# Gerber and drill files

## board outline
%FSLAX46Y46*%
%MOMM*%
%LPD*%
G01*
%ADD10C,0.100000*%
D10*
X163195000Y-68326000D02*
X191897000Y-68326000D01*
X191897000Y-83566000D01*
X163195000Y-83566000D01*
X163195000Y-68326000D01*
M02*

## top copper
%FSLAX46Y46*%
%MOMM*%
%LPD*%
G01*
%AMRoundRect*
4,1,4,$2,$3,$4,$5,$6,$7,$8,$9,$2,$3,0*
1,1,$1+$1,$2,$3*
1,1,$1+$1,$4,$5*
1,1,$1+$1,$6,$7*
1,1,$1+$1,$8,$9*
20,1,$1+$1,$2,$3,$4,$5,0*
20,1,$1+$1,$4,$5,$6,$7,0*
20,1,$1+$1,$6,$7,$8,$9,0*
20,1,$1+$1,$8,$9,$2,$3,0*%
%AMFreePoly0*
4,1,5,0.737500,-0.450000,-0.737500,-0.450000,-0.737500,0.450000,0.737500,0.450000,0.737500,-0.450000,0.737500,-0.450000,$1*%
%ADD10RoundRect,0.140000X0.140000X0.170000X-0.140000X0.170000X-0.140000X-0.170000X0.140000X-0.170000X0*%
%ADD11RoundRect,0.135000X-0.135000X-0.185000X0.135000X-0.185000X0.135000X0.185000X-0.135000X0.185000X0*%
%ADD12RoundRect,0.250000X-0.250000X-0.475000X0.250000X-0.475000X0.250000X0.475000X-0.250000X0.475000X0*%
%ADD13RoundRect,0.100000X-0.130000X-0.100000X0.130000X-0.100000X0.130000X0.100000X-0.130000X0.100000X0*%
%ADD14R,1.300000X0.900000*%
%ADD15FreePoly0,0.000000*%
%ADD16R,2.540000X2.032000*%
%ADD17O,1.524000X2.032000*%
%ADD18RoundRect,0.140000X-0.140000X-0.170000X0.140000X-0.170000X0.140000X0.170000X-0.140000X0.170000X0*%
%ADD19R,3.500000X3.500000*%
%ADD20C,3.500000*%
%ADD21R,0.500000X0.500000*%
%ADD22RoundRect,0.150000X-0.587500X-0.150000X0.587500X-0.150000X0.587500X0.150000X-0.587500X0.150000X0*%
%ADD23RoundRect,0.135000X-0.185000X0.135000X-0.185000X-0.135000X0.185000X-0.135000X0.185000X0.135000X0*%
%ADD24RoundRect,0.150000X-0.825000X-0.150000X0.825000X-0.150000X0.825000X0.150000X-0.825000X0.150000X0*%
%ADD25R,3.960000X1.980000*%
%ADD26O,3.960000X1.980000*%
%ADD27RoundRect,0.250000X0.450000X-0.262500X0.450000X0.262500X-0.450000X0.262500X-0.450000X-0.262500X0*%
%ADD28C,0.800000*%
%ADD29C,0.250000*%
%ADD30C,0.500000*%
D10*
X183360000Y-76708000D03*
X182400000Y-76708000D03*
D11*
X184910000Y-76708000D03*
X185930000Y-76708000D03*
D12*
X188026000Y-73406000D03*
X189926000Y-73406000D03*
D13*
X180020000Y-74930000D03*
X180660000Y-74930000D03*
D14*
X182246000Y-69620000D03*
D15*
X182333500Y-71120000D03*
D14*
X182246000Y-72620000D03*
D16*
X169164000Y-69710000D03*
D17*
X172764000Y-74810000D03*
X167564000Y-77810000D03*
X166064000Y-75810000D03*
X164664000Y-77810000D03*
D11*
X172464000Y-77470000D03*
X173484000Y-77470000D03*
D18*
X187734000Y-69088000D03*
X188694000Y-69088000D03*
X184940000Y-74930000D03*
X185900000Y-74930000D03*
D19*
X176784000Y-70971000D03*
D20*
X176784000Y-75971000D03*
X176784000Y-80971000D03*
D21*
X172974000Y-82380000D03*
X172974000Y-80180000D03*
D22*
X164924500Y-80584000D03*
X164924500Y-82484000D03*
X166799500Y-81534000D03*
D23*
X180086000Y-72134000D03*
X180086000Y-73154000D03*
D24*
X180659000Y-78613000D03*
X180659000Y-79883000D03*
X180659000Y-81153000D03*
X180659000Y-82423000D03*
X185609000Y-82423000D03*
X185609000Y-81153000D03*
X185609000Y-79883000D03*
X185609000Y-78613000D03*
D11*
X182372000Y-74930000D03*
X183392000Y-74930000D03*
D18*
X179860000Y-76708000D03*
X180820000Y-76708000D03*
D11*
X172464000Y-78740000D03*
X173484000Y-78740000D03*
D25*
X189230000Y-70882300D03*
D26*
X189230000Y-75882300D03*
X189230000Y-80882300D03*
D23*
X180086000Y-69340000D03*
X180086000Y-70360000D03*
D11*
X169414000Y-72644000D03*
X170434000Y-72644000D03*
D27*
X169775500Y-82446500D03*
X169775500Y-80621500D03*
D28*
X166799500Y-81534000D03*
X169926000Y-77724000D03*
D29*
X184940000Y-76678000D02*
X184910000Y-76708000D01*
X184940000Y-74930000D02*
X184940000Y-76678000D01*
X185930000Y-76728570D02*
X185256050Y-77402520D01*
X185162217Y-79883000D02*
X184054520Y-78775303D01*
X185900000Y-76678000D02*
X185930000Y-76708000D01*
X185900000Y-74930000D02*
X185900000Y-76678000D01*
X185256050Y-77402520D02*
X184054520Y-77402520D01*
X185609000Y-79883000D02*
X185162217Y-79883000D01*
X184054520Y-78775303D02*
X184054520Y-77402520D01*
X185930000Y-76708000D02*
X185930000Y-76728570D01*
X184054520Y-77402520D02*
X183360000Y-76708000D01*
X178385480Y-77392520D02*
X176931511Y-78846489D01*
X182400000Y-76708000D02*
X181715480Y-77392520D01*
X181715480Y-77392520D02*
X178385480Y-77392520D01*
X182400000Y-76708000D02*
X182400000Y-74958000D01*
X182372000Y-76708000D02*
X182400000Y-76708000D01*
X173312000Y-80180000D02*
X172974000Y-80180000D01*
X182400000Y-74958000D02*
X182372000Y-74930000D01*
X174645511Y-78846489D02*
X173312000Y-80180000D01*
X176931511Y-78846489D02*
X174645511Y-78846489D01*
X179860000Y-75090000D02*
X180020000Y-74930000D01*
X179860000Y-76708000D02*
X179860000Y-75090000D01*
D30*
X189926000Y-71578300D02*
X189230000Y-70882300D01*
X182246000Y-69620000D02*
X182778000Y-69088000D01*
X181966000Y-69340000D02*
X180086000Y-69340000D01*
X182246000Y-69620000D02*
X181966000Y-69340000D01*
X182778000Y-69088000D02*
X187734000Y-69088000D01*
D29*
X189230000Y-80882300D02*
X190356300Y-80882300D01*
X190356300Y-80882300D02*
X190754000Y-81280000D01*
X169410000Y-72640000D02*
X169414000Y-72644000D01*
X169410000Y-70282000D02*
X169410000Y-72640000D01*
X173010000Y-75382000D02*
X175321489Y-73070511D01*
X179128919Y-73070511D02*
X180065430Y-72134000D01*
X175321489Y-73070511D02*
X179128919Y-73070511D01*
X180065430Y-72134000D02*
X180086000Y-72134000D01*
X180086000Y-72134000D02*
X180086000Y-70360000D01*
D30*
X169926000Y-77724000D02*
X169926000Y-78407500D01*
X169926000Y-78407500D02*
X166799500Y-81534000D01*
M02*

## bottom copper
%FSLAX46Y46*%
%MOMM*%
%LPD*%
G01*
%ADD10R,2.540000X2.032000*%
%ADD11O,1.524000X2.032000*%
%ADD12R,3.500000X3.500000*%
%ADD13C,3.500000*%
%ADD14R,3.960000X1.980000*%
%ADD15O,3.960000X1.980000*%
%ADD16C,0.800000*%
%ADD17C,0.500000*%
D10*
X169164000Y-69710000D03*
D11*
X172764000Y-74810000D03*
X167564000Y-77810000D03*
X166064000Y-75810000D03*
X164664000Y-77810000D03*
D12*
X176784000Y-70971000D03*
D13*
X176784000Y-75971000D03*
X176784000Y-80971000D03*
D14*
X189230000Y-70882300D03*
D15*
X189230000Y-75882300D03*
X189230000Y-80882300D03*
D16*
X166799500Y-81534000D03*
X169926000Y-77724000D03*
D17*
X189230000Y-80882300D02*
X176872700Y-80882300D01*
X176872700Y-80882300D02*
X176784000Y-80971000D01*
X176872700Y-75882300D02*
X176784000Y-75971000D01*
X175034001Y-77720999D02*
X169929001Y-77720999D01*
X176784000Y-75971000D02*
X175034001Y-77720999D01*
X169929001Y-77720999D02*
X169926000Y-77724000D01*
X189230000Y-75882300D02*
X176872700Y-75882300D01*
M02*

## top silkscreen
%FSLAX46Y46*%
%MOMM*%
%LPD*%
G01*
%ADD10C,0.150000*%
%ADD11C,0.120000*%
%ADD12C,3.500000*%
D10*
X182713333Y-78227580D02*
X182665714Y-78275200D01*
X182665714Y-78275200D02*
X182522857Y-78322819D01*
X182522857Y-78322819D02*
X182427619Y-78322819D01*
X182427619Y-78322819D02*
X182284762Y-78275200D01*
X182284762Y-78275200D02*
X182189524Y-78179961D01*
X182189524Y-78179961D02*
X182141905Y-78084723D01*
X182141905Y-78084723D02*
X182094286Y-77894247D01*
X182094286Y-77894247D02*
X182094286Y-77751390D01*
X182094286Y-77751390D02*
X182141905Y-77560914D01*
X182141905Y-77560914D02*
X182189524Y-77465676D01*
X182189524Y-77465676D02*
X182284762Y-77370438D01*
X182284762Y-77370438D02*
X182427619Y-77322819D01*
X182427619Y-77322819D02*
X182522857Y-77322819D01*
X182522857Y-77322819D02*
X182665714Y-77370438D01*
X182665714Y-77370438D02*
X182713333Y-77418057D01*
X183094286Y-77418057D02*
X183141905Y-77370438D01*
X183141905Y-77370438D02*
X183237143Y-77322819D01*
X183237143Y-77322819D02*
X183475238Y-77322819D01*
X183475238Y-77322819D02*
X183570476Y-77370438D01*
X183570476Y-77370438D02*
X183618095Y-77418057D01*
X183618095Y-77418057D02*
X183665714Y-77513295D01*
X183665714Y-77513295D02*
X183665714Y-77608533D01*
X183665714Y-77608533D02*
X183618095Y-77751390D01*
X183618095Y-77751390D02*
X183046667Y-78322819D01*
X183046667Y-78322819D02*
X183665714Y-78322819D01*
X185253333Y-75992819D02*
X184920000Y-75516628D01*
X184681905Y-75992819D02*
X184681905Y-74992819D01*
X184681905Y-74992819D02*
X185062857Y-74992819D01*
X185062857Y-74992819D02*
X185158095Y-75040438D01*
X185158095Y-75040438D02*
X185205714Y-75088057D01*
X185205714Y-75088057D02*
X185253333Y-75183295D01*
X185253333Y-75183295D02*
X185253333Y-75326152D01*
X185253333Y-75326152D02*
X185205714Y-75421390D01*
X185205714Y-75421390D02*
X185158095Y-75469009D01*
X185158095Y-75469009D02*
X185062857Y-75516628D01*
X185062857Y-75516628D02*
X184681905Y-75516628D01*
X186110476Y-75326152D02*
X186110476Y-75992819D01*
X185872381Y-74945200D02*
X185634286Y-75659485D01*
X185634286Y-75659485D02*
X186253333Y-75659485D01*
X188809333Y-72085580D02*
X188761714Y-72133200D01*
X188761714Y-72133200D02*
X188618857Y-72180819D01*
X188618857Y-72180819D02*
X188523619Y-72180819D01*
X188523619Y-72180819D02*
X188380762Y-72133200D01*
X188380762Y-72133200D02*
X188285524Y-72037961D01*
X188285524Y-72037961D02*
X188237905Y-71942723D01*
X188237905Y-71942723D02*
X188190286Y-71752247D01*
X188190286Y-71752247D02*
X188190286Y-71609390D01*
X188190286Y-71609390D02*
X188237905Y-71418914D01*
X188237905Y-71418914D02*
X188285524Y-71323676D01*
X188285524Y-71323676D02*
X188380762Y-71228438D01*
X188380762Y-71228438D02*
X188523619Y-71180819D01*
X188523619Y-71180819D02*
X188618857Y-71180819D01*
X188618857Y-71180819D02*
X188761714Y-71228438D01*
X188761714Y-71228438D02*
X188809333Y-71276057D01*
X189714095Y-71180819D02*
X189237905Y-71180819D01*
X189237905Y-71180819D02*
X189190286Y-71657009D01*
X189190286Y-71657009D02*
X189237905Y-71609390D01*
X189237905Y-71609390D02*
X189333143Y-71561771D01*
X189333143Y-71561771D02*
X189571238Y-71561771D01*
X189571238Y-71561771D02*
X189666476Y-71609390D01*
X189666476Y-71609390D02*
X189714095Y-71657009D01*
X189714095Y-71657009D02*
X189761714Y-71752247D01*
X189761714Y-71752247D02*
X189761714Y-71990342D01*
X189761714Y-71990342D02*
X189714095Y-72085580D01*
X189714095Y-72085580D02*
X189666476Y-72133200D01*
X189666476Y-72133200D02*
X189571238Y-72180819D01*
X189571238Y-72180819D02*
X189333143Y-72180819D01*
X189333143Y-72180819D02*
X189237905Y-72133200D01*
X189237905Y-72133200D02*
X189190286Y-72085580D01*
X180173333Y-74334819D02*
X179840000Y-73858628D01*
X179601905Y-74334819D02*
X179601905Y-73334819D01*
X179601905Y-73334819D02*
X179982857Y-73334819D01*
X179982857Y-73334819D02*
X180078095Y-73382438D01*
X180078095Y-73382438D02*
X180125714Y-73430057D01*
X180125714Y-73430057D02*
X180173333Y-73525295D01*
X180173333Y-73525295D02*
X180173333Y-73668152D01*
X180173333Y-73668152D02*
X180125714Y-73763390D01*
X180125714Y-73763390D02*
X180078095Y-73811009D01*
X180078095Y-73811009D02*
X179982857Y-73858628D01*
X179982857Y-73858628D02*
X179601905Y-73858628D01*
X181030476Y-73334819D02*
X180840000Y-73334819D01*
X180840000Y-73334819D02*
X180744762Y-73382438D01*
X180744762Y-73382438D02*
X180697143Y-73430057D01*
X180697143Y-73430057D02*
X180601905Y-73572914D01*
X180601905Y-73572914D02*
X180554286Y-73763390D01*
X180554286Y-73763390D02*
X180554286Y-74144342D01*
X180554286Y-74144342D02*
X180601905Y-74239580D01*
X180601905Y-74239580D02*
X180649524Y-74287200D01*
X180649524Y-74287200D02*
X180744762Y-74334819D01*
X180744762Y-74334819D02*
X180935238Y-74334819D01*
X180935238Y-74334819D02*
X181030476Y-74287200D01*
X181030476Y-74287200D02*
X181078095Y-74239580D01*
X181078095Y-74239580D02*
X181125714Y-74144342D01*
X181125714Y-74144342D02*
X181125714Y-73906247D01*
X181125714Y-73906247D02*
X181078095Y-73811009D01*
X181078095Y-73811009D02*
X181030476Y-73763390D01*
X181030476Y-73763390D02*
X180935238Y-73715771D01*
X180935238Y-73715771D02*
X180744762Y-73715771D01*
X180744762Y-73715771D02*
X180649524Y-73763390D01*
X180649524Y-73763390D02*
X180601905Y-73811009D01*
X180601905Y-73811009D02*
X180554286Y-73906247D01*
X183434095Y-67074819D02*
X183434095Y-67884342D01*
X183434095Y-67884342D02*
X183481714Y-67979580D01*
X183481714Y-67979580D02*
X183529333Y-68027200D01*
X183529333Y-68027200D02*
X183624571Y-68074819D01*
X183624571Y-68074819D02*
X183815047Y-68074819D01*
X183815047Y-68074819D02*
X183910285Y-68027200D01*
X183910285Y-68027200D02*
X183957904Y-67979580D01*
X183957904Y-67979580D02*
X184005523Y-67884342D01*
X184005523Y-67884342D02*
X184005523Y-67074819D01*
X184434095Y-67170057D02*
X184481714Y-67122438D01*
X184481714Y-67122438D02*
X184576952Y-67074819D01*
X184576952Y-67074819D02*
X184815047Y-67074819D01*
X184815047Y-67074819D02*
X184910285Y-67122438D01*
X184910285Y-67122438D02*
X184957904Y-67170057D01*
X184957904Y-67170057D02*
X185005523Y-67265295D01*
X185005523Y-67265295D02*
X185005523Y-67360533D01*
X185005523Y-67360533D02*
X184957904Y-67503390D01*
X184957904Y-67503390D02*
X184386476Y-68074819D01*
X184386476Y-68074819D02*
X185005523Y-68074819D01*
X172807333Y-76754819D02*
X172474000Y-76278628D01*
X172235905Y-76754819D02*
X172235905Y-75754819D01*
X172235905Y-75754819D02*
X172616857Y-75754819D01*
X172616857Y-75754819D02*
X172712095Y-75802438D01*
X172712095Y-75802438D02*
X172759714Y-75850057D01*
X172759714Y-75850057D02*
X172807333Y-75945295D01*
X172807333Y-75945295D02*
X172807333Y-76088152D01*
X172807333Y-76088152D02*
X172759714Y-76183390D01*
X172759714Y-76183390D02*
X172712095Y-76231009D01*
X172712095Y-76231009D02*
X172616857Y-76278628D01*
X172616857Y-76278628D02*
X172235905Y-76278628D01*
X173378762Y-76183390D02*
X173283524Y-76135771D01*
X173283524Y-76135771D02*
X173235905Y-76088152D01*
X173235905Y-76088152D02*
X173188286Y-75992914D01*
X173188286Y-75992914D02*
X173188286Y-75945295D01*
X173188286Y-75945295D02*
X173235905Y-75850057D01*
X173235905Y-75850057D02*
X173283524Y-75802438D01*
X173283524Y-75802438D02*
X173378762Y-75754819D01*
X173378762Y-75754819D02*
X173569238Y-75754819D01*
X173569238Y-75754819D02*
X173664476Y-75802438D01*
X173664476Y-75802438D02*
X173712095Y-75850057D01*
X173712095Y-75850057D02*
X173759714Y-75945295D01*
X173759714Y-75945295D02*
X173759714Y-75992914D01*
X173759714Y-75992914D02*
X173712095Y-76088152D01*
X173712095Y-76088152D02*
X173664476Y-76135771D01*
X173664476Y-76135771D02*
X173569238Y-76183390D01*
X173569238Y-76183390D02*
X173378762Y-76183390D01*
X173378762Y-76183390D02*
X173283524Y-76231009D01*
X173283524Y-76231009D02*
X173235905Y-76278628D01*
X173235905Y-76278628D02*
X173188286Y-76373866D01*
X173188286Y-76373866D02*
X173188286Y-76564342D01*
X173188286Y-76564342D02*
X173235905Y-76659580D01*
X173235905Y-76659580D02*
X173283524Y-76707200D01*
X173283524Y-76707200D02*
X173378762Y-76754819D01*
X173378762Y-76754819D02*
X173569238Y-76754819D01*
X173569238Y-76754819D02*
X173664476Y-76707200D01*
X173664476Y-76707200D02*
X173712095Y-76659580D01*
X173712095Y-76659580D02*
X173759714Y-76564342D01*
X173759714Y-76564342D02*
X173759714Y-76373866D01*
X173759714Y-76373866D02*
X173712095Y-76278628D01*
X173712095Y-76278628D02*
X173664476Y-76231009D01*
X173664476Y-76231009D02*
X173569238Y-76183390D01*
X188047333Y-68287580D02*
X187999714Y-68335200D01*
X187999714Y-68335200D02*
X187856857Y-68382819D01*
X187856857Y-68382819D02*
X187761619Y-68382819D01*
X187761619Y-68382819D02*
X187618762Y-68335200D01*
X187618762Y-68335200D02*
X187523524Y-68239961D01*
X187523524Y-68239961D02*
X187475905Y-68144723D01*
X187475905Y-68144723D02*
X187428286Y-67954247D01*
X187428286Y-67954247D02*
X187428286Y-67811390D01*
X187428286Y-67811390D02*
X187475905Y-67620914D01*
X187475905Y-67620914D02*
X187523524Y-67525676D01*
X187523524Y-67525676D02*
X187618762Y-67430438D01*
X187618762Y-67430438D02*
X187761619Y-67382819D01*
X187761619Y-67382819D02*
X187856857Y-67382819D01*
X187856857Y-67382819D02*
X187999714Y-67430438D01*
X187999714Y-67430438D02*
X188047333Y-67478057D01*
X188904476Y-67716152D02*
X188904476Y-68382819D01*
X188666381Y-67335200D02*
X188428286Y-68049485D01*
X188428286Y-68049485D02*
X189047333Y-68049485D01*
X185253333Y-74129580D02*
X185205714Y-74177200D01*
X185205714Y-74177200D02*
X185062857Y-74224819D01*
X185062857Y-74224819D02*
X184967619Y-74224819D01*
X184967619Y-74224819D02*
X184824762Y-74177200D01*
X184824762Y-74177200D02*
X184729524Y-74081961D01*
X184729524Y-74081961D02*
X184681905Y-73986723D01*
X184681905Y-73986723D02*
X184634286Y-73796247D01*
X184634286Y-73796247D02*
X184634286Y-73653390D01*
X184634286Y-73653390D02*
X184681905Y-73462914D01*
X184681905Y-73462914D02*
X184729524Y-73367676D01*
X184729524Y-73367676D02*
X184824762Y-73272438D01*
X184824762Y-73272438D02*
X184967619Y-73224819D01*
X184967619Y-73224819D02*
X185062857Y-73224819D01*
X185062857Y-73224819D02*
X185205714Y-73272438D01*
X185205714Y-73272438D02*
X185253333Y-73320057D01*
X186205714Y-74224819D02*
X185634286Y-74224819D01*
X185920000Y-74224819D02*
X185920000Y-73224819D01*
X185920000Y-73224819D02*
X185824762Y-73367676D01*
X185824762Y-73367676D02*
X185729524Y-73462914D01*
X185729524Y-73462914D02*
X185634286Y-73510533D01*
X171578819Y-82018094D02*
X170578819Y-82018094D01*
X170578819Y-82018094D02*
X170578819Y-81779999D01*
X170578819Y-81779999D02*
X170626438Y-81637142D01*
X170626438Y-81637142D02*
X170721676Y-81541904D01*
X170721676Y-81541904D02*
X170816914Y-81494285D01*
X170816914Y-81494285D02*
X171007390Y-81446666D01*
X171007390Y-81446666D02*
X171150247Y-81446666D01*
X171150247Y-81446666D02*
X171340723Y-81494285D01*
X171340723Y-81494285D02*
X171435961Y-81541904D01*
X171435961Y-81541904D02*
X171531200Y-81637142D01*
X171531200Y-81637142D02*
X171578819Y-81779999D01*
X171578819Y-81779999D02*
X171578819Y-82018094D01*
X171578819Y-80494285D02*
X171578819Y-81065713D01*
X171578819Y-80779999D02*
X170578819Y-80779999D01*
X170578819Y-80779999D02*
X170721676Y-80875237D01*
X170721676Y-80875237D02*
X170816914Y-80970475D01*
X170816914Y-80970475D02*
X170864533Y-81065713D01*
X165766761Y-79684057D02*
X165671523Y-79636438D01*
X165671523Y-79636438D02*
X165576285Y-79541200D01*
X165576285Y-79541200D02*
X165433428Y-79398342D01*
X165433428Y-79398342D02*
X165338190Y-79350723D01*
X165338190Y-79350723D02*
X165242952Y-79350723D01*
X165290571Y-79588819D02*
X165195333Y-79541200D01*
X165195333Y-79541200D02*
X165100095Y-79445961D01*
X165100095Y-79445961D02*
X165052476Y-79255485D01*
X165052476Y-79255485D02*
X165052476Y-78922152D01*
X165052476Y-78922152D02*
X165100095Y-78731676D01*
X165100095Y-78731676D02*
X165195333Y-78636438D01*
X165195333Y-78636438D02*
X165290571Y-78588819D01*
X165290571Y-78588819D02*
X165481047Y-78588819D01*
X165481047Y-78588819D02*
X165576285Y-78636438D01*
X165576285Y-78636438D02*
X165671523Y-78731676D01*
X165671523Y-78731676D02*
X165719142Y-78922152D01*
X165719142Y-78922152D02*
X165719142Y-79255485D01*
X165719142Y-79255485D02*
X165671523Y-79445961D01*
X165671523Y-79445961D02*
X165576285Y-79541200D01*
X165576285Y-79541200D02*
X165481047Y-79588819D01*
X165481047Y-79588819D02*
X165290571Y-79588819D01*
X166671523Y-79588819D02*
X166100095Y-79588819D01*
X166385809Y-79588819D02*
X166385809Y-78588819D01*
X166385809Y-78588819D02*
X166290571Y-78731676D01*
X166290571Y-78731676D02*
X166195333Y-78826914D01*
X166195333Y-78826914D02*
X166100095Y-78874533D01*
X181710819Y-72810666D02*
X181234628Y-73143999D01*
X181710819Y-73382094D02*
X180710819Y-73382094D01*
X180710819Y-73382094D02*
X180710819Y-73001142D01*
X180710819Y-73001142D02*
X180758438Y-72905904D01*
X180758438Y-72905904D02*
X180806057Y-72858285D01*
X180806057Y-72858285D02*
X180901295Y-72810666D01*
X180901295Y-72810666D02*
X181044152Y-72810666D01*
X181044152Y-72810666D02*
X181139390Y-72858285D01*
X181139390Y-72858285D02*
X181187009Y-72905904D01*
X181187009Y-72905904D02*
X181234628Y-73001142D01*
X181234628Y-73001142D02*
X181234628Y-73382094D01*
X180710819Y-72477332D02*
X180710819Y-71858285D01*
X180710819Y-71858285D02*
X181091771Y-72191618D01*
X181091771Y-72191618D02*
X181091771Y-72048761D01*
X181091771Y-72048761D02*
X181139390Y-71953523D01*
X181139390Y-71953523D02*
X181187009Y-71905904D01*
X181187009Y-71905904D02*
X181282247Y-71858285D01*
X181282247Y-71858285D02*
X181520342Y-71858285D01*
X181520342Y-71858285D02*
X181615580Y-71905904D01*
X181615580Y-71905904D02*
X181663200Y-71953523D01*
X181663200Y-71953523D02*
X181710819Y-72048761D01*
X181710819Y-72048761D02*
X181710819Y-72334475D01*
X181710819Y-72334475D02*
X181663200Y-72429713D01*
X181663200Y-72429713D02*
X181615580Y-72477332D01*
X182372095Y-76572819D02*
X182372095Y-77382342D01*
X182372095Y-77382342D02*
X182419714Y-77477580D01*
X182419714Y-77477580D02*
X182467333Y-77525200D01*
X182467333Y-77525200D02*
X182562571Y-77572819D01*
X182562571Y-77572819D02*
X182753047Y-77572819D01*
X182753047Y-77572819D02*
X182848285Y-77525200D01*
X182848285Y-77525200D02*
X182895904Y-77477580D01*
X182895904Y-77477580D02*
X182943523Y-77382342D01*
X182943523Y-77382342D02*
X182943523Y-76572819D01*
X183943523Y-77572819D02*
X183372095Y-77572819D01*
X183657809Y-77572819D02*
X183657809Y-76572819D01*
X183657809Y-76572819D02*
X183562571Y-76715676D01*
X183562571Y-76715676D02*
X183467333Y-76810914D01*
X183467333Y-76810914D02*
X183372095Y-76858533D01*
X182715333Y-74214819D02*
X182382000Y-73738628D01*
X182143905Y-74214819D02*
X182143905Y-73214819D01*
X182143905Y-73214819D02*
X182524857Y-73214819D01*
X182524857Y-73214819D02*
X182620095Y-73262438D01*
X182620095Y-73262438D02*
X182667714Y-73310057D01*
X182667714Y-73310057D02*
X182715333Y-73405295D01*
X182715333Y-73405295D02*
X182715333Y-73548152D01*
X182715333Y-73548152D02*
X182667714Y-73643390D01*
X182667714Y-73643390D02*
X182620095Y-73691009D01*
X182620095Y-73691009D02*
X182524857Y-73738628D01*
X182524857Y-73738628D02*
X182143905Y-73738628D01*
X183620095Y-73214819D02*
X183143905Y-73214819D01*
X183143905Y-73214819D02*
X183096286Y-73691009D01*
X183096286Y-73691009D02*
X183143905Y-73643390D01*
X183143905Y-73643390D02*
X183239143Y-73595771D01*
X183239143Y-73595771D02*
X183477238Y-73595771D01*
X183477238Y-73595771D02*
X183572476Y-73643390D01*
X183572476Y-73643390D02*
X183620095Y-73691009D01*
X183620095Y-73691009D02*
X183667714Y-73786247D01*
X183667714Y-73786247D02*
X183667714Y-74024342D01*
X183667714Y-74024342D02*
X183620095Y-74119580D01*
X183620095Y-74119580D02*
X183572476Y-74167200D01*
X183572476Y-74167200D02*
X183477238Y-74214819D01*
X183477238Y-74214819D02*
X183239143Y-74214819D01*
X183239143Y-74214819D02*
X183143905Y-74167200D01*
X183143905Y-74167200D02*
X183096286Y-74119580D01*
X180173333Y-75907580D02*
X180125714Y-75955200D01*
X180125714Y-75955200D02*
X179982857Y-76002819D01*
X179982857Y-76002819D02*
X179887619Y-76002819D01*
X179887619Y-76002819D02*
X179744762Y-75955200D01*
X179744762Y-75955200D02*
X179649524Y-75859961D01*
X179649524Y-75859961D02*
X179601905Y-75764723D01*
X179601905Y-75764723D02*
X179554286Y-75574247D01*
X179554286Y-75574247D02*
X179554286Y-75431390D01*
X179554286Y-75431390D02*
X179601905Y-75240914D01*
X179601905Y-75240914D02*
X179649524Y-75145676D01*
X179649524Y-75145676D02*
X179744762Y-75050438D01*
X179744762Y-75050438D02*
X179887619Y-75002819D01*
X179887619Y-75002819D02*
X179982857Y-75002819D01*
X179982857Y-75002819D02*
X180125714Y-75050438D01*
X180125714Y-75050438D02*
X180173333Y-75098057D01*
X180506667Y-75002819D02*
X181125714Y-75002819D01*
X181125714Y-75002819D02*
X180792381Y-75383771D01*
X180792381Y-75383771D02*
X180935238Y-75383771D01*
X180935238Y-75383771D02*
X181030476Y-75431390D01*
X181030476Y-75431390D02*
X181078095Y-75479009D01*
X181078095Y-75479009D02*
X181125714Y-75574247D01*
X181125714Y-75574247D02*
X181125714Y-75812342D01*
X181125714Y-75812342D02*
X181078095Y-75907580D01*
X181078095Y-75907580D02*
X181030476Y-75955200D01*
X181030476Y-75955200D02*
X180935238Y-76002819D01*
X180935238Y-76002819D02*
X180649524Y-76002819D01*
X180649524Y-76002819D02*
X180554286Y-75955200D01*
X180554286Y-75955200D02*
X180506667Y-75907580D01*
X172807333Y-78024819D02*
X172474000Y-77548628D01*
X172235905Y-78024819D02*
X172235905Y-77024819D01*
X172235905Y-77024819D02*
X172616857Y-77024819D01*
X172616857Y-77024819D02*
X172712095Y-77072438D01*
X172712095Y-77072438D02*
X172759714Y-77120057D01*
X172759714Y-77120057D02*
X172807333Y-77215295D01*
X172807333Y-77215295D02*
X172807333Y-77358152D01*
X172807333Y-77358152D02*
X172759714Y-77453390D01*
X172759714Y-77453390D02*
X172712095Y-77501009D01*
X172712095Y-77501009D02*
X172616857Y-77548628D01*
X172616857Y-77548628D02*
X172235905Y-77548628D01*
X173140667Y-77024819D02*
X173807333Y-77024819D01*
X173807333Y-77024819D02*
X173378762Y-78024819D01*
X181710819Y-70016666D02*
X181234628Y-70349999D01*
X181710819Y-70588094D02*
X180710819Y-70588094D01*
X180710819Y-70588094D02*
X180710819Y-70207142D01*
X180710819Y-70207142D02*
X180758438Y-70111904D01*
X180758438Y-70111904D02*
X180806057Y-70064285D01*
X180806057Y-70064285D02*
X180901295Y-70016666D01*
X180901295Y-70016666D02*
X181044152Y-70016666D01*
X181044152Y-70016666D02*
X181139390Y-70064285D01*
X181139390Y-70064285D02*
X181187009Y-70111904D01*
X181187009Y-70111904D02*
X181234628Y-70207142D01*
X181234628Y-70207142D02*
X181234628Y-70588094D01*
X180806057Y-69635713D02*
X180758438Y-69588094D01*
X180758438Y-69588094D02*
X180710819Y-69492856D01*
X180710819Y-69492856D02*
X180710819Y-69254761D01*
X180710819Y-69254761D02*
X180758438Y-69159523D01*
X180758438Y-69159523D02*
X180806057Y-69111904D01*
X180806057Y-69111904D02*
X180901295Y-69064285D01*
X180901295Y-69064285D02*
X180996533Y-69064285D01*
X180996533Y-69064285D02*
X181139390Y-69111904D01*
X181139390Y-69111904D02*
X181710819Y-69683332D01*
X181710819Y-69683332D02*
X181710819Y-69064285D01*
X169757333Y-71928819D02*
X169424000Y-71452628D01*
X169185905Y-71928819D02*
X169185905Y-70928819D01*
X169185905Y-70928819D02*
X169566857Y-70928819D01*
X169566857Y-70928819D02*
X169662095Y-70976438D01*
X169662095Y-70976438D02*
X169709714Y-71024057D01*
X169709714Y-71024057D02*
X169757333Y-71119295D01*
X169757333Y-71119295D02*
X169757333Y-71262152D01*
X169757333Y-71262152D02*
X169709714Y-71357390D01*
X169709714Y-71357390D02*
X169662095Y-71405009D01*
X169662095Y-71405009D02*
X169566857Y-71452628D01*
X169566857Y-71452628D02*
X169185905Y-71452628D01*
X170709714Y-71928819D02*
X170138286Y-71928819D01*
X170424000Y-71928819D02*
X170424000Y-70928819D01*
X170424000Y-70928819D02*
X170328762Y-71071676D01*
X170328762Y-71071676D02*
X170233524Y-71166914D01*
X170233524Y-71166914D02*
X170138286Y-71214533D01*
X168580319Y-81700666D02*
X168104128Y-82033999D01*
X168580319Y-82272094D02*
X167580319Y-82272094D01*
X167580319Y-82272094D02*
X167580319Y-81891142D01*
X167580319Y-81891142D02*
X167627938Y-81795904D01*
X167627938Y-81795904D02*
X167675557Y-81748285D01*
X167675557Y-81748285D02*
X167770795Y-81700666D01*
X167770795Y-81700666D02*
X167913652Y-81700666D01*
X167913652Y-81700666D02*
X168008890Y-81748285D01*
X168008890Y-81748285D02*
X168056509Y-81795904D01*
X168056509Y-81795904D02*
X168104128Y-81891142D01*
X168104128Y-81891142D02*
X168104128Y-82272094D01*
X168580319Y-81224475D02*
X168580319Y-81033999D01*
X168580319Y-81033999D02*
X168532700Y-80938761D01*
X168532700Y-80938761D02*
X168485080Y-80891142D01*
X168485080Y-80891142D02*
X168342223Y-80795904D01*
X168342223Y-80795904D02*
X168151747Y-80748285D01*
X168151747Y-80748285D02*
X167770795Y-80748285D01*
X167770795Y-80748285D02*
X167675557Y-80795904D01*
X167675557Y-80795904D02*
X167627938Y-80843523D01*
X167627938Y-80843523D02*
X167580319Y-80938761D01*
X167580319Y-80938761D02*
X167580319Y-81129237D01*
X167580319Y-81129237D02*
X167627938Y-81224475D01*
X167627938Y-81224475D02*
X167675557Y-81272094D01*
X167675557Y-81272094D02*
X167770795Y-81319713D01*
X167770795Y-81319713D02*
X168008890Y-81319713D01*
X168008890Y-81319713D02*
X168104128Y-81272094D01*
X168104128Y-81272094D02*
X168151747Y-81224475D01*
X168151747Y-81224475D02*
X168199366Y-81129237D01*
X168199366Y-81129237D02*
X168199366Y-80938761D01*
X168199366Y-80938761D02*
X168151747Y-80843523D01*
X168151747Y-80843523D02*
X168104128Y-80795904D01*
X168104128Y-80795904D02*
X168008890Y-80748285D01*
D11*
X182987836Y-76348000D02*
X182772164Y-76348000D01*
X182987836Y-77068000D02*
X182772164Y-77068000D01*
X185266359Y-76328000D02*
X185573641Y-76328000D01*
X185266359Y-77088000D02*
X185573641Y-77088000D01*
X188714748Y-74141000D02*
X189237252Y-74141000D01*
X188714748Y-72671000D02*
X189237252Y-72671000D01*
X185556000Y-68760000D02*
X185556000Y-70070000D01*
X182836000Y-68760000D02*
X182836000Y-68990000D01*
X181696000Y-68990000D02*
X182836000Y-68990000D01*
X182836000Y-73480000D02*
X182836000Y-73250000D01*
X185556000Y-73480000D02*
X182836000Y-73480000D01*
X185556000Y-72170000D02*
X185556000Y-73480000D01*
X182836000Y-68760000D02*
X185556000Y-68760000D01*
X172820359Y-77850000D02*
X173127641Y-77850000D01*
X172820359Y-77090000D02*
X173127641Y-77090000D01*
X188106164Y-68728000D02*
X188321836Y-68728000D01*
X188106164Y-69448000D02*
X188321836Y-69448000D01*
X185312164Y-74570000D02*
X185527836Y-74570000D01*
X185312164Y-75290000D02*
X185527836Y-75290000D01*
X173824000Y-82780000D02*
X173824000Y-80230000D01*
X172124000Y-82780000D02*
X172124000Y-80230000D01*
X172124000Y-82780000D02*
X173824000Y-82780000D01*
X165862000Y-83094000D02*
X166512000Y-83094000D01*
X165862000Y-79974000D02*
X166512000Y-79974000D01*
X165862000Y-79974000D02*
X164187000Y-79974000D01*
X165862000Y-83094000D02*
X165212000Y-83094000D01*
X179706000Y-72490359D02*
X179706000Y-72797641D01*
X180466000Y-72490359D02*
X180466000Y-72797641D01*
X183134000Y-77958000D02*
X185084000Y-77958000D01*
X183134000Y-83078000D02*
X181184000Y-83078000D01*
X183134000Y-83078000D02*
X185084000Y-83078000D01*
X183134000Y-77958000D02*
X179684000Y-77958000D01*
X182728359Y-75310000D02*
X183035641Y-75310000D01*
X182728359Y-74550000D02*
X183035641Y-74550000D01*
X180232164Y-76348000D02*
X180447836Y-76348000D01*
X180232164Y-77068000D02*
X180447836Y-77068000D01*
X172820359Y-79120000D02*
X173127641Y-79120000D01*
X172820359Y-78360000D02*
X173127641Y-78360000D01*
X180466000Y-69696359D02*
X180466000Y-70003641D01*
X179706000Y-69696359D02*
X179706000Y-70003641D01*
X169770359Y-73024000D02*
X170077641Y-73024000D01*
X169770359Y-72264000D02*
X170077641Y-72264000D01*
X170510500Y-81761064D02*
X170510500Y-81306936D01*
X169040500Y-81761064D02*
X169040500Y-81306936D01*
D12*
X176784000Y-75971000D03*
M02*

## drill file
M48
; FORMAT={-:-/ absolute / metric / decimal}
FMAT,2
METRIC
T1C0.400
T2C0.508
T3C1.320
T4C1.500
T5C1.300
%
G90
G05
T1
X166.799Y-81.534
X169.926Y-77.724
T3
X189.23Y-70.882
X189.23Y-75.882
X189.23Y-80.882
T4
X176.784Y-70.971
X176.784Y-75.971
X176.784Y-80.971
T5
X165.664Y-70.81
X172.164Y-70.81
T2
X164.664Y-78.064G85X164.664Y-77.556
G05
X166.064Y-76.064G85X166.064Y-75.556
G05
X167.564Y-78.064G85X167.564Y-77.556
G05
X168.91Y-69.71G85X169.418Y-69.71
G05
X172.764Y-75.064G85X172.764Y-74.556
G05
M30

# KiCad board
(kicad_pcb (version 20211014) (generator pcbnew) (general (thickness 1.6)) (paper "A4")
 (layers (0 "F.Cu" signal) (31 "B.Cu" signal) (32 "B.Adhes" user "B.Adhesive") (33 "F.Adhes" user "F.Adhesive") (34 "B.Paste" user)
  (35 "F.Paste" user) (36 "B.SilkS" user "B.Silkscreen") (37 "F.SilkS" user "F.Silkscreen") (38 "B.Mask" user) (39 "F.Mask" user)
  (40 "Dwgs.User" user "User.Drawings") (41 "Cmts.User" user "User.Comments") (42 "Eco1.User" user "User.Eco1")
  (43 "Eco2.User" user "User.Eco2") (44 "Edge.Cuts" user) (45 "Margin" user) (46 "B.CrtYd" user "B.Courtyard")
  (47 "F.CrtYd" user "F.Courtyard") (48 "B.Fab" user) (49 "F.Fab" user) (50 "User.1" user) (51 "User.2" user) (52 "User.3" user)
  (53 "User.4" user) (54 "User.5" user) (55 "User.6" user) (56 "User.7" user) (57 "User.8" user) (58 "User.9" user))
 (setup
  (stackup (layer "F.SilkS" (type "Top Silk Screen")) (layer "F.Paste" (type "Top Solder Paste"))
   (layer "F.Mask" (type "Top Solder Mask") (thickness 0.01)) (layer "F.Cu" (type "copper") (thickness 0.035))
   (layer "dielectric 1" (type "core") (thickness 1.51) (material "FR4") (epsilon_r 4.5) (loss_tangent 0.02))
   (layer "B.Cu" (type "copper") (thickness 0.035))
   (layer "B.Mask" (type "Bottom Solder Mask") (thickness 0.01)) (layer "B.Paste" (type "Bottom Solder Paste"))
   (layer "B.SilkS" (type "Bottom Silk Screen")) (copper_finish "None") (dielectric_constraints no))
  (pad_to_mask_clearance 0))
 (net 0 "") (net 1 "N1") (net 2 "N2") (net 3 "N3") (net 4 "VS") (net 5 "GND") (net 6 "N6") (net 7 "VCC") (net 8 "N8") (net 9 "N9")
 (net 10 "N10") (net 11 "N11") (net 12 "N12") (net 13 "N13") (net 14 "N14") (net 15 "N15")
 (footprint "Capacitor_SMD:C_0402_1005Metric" (layer "F.Cu") (at 182.88 76.708 180)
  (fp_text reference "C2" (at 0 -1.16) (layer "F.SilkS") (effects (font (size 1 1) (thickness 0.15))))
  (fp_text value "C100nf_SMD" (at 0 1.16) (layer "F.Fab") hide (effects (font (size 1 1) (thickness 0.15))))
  (fp_line (start -0.107836 0.36) (end 0.107836 0.36) (layer "F.SilkS") (width 0.12))
  (fp_line (start -0.107836 -0.36) (end 0.107836 -0.36) (layer "F.SilkS") (width 0.12))
  (pad "1" smd roundrect locked (at -0.48 0 180) (size 0.56 0.62) (layers "F.Cu" "F.Paste" "F.Mask") (roundrect_rratio 0.25) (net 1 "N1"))
  (pad "2" smd roundrect locked (at 0.48 0 180) (size 0.56 0.62) (layers "F.Cu" "F.Paste" "F.Mask") (roundrect_rratio 0.25) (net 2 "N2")))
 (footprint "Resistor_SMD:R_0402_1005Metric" (layer "F.Cu") (at 185.42 76.708)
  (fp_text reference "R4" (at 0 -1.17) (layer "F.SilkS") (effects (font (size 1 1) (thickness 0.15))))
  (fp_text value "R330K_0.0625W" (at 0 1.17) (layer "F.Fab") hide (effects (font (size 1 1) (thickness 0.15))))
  (fp_line (start -0.153641 -0.38) (end 0.153641 -0.38) (layer "F.SilkS") (width 0.12))
  (fp_line (start -0.153641 0.38) (end 0.153641 0.38) (layer "F.SilkS") (width 0.12))
  (pad "1" smd roundrect locked (at -0.51 0) (size 0.54 0.64) (layers "F.Cu" "F.Paste" "F.Mask") (roundrect_rratio 0.25) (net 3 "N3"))
  (pad "2" smd roundrect locked (at 0.51 0) (size 0.54 0.64) (layers "F.Cu" "F.Paste" "F.Mask") (roundrect_rratio 0.25) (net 1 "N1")))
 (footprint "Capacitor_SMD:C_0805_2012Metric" (layer "F.Cu") (at 188.976 73.406)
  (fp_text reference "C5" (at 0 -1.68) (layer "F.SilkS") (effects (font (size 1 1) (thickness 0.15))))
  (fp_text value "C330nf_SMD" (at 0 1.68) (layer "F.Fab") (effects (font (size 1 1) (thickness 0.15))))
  (fp_line (start -0.261252 0.735) (end 0.261252 0.735) (layer "F.SilkS") (width 0.12))
  (fp_line (start -0.261252 -0.735) (end 0.261252 -0.735) (layer "F.SilkS") (width 0.12))
  (pad "1" smd roundrect locked (at -0.95 0) (size 1 1.45) (layers "F.Cu" "F.Paste" "F.Mask") (roundrect_rratio 0.25) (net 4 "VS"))
  (pad "2" smd roundrect locked (at 0.95 0) (size 1 1.45) (layers "F.Cu" "F.Paste" "F.Mask") (roundrect_rratio 0.25) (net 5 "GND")))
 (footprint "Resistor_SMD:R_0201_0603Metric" (layer "F.Cu") (at 180.34 74.93)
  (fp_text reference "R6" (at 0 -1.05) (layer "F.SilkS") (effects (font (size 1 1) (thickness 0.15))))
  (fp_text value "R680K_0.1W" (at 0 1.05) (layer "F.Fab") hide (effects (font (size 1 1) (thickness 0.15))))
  (pad "" smd roundrect locked (at 0.345 0) (size 0.318 0.36) (layers "F.Paste") (roundrect_rratio 0.25))
  (pad "" smd roundrect locked (at -0.345 0) (size 0.318 0.36) (layers "F.Paste") (roundrect_rratio 0.25))
  (pad "1" smd roundrect locked (at -0.32 0) (size 0.46 0.4) (layers "F.Cu" "F.Mask") (roundrect_rratio 0.25) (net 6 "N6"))
  (pad "2" smd roundrect locked (at 0.32 0) (size 0.46 0.4) (layers "F.Cu" "F.Mask") (roundrect_rratio 0.25) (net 5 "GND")))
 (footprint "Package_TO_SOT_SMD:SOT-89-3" (layer "F.Cu") (at 183.896 71.12)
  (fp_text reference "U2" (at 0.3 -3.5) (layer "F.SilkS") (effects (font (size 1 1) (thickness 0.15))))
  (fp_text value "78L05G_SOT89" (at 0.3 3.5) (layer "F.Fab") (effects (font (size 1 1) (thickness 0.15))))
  (fp_line (start 1.66 -2.36) (end 1.66 -1.05) (layer "F.SilkS") (width 0.12))
  (fp_line (start -1.06 -2.36) (end -1.06 -2.13) (layer "F.SilkS") (width 0.12))
  (fp_line (start -2.2 -2.13) (end -1.06 -2.13) (layer "F.SilkS") (width 0.12))
  (fp_line (start -1.06 2.36) (end -1.06 2.13) (layer "F.SilkS") (width 0.12))
  (fp_line (start 1.66 2.36) (end -1.06 2.36) (layer "F.SilkS") (width 0.12))
  (fp_line (start 1.66 1.05) (end 1.66 2.36) (layer "F.SilkS") (width 0.12))
  (fp_line (start -1.06 -2.36) (end 1.66 -2.36) (layer "F.SilkS") (width 0.12))
  (pad "1" smd rect locked (at -1.65 -1.5) (size 1.3 0.9) (layers "F.Cu" "F.Paste" "F.Mask") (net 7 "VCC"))
  (pad "2" smd custom locked (at -1.5625 0) (size 1.475 0.9) (layers "F.Cu" "F.Paste" "F.Mask") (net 5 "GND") (zone_connect 2)
   (options (clearance outline) (anchor rect)) (primitives))
  (pad "3" smd rect locked (at -1.65 1.5) (size 1.3 0.9) (layers "F.Cu" "F.Paste" "F.Mask") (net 4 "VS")))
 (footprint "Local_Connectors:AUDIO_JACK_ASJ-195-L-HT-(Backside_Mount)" (layer "F.Cu") (at 169.164 67.31 90)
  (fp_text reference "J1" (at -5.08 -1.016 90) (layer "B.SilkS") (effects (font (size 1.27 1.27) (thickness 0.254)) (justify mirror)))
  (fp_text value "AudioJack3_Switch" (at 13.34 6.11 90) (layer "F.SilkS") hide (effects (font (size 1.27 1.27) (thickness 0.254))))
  (pad "" np_thru_hole circle (at -3.5 -3.5 90) (size 1.3 1.3) (drill 1.3) (layers F&B.Cu *.Mask))
  (pad "" np_thru_hole circle (at -3.5 3 90) (size 1.3 1.3) (drill 1.3) (layers F&B.Cu *.Mask))
  (pad "1" thru_hole rect (at -2.4 0 90) (size 2.032 2.54) (drill oval 0.508 1.016) (layers *.Cu *.Mask) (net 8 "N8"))
  (pad "2" thru_hole oval (at -7.5 3.6 90) (size 2.032 1.524) (drill oval 1.016 0.508) (layers *.Cu *.Mask) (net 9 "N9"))
  (pad "3" thru_hole oval (at -10.5 -1.6 90) (size 2.032 1.524) (drill oval 1.016 0.508) (layers *.Cu *.Mask) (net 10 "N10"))
  (pad "5" thru_hole oval (at -8.5 -3.1 90) (size 2.032 1.524) (drill oval 1.016 0.508) (layers *.Cu *.Mask) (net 5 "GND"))
  (pad "6" thru_hole oval (at -10.5 -4.5 90) (size 2.032 1.524) (drill oval 1.016 0.508) (layers *.Cu *.Mask) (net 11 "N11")))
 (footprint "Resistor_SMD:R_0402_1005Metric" (layer "F.Cu") (at 172.974 77.47)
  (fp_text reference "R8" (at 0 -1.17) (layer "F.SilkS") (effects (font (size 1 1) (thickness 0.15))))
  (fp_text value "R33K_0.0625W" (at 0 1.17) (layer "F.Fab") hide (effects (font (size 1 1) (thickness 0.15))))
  (fp_line (start -0.153641 0.38) (end 0.153641 0.38) (layer "F.SilkS") (width 0.12))
  (fp_line (start -0.153641 -0.38) (end 0.153641 -0.38) (layer "F.SilkS") (width 0.12))
  (pad "1" smd roundrect locked (at -0.51 0) (size 0.54 0.64) (layers "F.Cu" "F.Paste" "F.Mask") (roundrect_rratio 0.25) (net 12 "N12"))
  (pad "2" smd roundrect locked (at 0.51 0) (size 0.54 0.64) (layers "F.Cu" "F.Paste" "F.Mask") (roundrect_rratio 0.25) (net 5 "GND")))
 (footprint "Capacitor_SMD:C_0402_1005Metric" (layer "F.Cu") (at 188.214 69.088)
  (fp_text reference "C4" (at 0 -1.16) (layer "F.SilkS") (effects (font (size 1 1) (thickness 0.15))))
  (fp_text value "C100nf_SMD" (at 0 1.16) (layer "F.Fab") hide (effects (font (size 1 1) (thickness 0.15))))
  (fp_line (start -0.107836 -0.36) (end 0.107836 -0.36) (layer "F.SilkS") (width 0.12))
  (fp_line (start -0.107836 0.36) (end 0.107836 0.36) (layer "F.SilkS") (width 0.12))
  (pad "1" smd roundrect locked (at -0.48 0) (size 0.56 0.62) (layers "F.Cu" "F.Paste" "F.Mask") (roundrect_rratio 0.25) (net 7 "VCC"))
  (pad "2" smd roundrect locked (at 0.48 0) (size 0.56 0.62) (layers "F.Cu" "F.Paste" "F.Mask") (roundrect_rratio 0.25) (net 5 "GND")))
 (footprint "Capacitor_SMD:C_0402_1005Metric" (layer "F.Cu") (at 185.42 74.93)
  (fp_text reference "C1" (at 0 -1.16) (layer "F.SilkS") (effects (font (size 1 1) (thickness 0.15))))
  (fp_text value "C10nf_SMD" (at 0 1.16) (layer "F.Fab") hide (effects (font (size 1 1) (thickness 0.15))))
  (fp_line (start -0.107836 -0.36) (end 0.107836 -0.36) (layer "F.SilkS") (width 0.12))
  (fp_line (start -0.107836 0.36) (end 0.107836 0.36) (layer "F.SilkS") (width 0.12))
  (pad "1" smd roundrect locked (at -0.48 0) (size 0.56 0.62) (layers "F.Cu" "F.Paste" "F.Mask") (roundrect_rratio 0.25) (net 3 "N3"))
  (pad "2" smd roundrect locked (at 0.48 0) (size 0.56 0.62) (layers "F.Cu" "F.Paste" "F.Mask") (roundrect_rratio 0.25) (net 1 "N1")))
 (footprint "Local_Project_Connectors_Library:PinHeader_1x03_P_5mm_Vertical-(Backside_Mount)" (layer "F.Cu") (at 176.784 70.971)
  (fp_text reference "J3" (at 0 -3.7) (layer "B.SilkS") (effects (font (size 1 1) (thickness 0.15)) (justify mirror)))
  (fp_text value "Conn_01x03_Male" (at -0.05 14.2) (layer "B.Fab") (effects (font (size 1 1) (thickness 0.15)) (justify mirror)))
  (pad "1" thru_hole rect (at 0 0) (size 3.5 3.5) (drill 1.5) (layers *.Cu *.Mask) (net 5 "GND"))
  (pad "2" thru_hole circle (at 0 5) (size 3.5 3.5) (drill 1.5) (layers *.Cu *.Mask "F.SilkS") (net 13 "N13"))
  (pad "3" thru_hole circle (at 0 10) (size 3.5 3.5) (drill 1.5) (layers *.Cu *.Mask) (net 4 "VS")))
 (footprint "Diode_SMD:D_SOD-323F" (layer "F.Cu") (at 172.974 81.28 90)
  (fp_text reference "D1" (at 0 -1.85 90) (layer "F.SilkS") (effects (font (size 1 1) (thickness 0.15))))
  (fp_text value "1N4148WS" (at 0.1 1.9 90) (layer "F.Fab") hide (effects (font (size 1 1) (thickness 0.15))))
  (fp_line (start -1.5 0.85) (end 1.05 0.85) (layer "F.SilkS") (width 0.12))
  (fp_line (start -1.5 -0.85) (end 1.05 -0.85) (layer "F.SilkS") (width 0.12))
  (fp_line (start -1.5 -0.85) (end -1.5 0.85) (layer "F.SilkS") (width 0.12))
  (pad "1" smd rect locked (at -1.1 0 90) (size 0.5 0.5) (layers "F.Cu" "F.Paste" "F.Mask") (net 6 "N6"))
  (pad "2" smd rect locked (at 1.1 0 90) (size 0.5 0.5) (layers "F.Cu" "F.Paste" "F.Mask") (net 2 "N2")))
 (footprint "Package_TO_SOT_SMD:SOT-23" (layer "F.Cu") (at 165.862 81.534)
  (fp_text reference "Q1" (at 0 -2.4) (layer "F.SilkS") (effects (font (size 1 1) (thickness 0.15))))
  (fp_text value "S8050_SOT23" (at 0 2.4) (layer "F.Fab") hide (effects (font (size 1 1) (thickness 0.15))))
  (fp_line (start 0 1.56) (end 0.65 1.56) (layer "F.SilkS") (width 0.12))
  (fp_line (start 0 -1.56) (end 0.65 -1.56) (layer "F.SilkS") (width 0.12))
  (fp_line (start 0 -1.56) (end -1.675 -1.56) (layer "F.SilkS") (width 0.12))
  (fp_line (start 0 1.56) (end -0.65 1.56) (layer "F.SilkS") (width 0.12))
  (pad "1" smd roundrect locked (at -0.9375 -0.95) (size 1.475 0.6) (layers "F.Cu" "F.Paste" "F.Mask") (roundrect_rratio 0.25)
   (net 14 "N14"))
  (pad "2" smd roundrect locked (at -0.9375 0.95) (size 1.475 0.6) (layers "F.Cu" "F.Paste" "F.Mask") (roundrect_rratio 0.25) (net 5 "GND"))
  (pad "3" smd roundrect locked (at 0.9375 0) (size 1.475 0.6) (layers "F.Cu" "F.Paste" "F.Mask") (roundrect_rratio 0.25) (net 13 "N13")))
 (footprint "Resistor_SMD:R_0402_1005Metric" (layer "F.Cu") (at 180.086 72.644 -90)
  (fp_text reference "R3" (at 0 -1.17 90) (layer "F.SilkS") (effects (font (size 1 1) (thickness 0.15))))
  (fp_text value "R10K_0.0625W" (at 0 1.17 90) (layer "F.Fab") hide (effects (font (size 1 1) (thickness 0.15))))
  (fp_line (start -0.153641 0.38) (end 0.153641 0.38) (layer "F.SilkS") (width 0.12))
  (fp_line (start -0.153641 -0.38) (end 0.153641 -0.38) (layer "F.SilkS") (width 0.12))
  (pad "1" smd roundrect locked (at -0.51 0 270) (size 0.54 0.64) (layers "F.Cu" "F.Paste" "F.Mask") (roundrect_rratio 0.25) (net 9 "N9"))
  (pad "2" smd roundrect locked (at 0.51 0 270) (size 0.54 0.64) (layers "F.Cu" "F.Paste" "F.Mask") (roundrect_rratio 0.25) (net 5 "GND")))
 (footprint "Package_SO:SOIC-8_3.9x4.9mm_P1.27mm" (layer "F.Cu") (at 183.134 80.518)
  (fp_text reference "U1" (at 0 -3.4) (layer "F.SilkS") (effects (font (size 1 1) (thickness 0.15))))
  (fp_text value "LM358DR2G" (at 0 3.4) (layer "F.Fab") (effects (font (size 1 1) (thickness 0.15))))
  (fp_line (start 0 -2.56) (end 1.95 -2.56) (layer "F.SilkS") (width 0.12))
  (fp_line (start 0 2.56) (end -1.95 2.56) (layer "F.SilkS") (width 0.12))
  (fp_line (start 0 2.56) (end 1.95 2.56) (layer "F.SilkS") (width 0.12))
  (fp_line (start 0 -2.56) (end -3.45 -2.56) (layer "F.SilkS") (width 0.12))
  (pad "1" smd roundrect locked (at -2.475 -1.905) (size 1.95 0.6) (layers "F.Cu" "F.Paste" "F.Mask") (roundrect_rratio 0.25) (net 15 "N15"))
  (pad "2" smd roundrect locked (at -2.475 -0.635) (size 1.95 0.6) (layers "F.Cu" "F.Paste" "F.Mask") (roundrect_rratio 0.25) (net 12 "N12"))
  (pad "3" smd roundrect locked (at -2.475 0.635) (size 1.95 0.6) (layers "F.Cu" "F.Paste" "F.Mask") (roundrect_rratio 0.25) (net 6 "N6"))
  (pad "4" smd roundrect locked (at -2.475 1.905) (size 1.95 0.6) (layers "F.Cu" "F.Paste" "F.Mask") (roundrect_rratio 0.25) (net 5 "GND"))
  (pad "5" smd roundrect locked (at 2.475 1.905) (size 1.95 0.6) (layers "F.Cu" "F.Paste" "F.Mask") (roundrect_rratio 0.25) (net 3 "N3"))
  (pad "6" smd roundrect locked (at 2.475 0.635) (size 1.95 0.6) (layers "F.Cu" "F.Paste" "F.Mask") (roundrect_rratio 0.25) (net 9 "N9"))
  (pad "7" smd roundrect locked (at 2.475 -0.635) (size 1.95 0.6) (layers "F.Cu" "F.Paste" "F.Mask") (roundrect_rratio 0.25) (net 1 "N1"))
  (pad "8" smd roundrect locked (at 2.475 -1.905) (size 1.95 0.6) (layers "F.Cu" "F.Paste" "F.Mask") (roundrect_rratio 0.25) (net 7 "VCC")))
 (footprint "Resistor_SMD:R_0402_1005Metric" (layer "F.Cu") (at 182.882 74.93)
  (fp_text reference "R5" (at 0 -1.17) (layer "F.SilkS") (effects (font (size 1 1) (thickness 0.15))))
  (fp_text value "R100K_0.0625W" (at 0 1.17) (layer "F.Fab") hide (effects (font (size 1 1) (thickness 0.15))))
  (fp_line (start -0.153641 0.38) (end 0.153641 0.38) (layer "F.SilkS") (width 0.12))
  (fp_line (start -0.153641 -0.38) (end 0.153641 -0.38) (layer "F.SilkS") (width 0.12))
  (pad "1" smd roundrect locked (at -0.51 0) (size 0.54 0.64) (layers "F.Cu" "F.Paste" "F.Mask") (roundrect_rratio 0.25) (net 2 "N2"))
  (pad "2" smd roundrect locked (at 0.51 0) (size 0.54 0.64) (layers "F.Cu" "F.Paste" "F.Mask") (roundrect_rratio 0.25) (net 5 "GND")))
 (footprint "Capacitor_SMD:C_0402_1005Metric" (layer "F.Cu") (at 180.34 76.708)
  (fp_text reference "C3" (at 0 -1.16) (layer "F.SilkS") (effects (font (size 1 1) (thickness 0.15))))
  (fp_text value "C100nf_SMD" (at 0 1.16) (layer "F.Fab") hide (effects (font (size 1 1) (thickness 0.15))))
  (fp_line (start -0.107836 -0.36) (end 0.107836 -0.36) (layer "F.SilkS") (width 0.12))
  (fp_line (start -0.107836 0.36) (end 0.107836 0.36) (layer "F.SilkS") (width 0.12))
  (pad "1" smd roundrect locked (at -0.48 0) (size 0.56 0.62) (layers "F.Cu" "F.Paste" "F.Mask") (roundrect_rratio 0.25) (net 6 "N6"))
  (pad "2" smd roundrect locked (at 0.48 0) (size 0.56 0.62) (layers "F.Cu" "F.Paste" "F.Mask") (roundrect_rratio 0.25) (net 5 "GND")))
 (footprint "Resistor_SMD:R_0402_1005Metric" (layer "F.Cu") (at 172.974 78.74)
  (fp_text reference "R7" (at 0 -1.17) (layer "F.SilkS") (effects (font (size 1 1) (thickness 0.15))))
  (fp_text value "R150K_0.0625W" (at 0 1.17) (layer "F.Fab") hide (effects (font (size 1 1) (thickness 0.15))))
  (fp_line (start -0.153641 0.38) (end 0.153641 0.38) (layer "F.SilkS") (width 0.12))
  (fp_line (start -0.153641 -0.38) (end 0.153641 -0.38) (layer "F.SilkS") (width 0.12))
  (pad "1" smd roundrect locked (at -0.51 0) (size 0.54 0.64) (layers "F.Cu" "F.Paste" "F.Mask") (roundrect_rratio 0.25) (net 7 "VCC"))
  (pad "2" smd roundrect locked (at 0.51 0) (size 0.54 0.64) (layers "F.Cu" "F.Paste" "F.Mask") (roundrect_rratio 0.25) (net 12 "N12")))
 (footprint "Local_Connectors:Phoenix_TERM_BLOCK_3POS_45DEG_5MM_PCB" (layer "F.Cu") (at 189.23 70.8823 -90)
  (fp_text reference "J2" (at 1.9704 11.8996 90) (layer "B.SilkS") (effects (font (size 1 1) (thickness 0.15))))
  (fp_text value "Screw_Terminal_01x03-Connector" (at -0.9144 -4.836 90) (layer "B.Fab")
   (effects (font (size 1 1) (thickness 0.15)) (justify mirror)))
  (pad "1" thru_hole rect locked (at 0 0 270) (size 1.98 3.96) (drill 1.32) (layers *.Cu *.Mask "F.Paste") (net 5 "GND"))
  (pad "2" thru_hole oval locked (at 5 0 270) (size 1.98 3.96) (drill 1.32) (layers *.Cu *.Mask "F.Paste") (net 13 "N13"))
  (pad "3" thru_hole oval locked (at 10 0 270) (size 1.98 3.96) (drill 1.32) (layers *.Cu *.Mask "F.Paste") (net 4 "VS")))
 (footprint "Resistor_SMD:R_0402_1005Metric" (layer "F.Cu") (at 180.086 69.85 -90)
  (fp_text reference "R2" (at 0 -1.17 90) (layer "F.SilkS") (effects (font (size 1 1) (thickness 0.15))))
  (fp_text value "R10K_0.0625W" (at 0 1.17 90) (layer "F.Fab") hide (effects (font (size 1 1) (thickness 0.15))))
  (fp_line (start -0.153641 -0.38) (end 0.153641 -0.38) (layer "F.SilkS") (width 0.12))
  (fp_line (start -0.153641 0.38) (end 0.153641 0.38) (layer "F.SilkS") (width 0.12))
  (pad "1" smd roundrect locked (at -0.51 0 270) (size 0.54 0.64) (layers "F.Cu" "F.Paste" "F.Mask") (roundrect_rratio 0.25) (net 7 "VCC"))
  (pad "2" smd roundrect locked (at 0.51 0 270) (size 0.54 0.64) (layers "F.Cu" "F.Paste" "F.Mask") (roundrect_rratio 0.25) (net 9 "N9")))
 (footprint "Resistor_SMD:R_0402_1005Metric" (layer "F.Cu") (at 169.924 72.644)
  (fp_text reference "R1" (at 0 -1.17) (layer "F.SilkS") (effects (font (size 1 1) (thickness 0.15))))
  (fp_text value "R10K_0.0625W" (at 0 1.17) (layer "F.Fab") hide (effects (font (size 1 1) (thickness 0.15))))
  (fp_line (start -0.153641 0.38) (end 0.153641 0.38) (layer "F.SilkS") (width 0.12))
  (fp_line (start -0.153641 -0.38) (end 0.153641 -0.38) (layer "F.SilkS") (width 0.12))
  (pad "1" smd roundrect locked (at -0.51 0) (size 0.54 0.64) (layers "F.Cu" "F.Paste" "F.Mask") (roundrect_rratio 0.25) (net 8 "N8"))
  (pad "2" smd roundrect locked (at 0.51 0) (size 0.54 0.64) (layers "F.Cu" "F.Paste" "F.Mask") (roundrect_rratio 0.25) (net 3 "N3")))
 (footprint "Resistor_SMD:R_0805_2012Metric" (layer "F.Cu") (at 169.7755 81.534 90)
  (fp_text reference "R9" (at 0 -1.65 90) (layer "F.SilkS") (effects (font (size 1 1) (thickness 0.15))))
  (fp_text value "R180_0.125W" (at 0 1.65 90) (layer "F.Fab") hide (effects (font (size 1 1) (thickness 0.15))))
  (fp_line (start -0.227064 0.735) (end 0.227064 0.735) (layer "F.SilkS") (width 0.12))
  (fp_line (start -0.227064 -0.735) (end 0.227064 -0.735) (layer "F.SilkS") (width 0.12))
  (pad "1" smd roundrect locked (at -0.9125 0 90) (size 1.025 1.4) (layers "F.Cu" "F.Paste" "F.Mask") (roundrect_rratio 0.243902)
   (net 15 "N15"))
  (pad "2" smd roundrect locked (at 0.9125 0 90) (size 1.025 1.4) (layers "F.Cu" "F.Paste" "F.Mask") (roundrect_rratio 0.243902)
   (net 14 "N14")))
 (gr_rect (start 191.897 83.566) (end 163.195 68.326) (layer "Edge.Cuts") (width 0.1) (fill none))
 (segment (start 184.94 76.678) (end 184.91 76.708) (width 0.25) (layer "F.Cu") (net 3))
 (segment (start 184.94 74.93) (end 184.94 76.678) (width 0.25) (layer "F.Cu") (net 3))
 (segment (start 185.93 76.72857) (end 185.25605 77.40252) (width 0.25) (layer "F.Cu") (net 1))
 (segment (start 185.162217 79.883) (end 184.05452 78.775303) (width 0.25) (layer "F.Cu") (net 1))
 (segment (start 185.9 76.678) (end 185.93 76.708) (width 0.25) (layer "F.Cu") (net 1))
 (segment (start 185.9 74.93) (end 185.9 76.678) (width 0.25) (layer "F.Cu") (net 1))
 (segment (start 185.25605 77.40252) (end 184.05452 77.40252) (width 0.25) (layer "F.Cu") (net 1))
 (segment (start 185.609 79.883) (end 185.162217 79.883) (width 0.25) (layer "F.Cu") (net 1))
 (segment (start 184.05452 78.775303) (end 184.05452 77.40252) (width 0.25) (layer "F.Cu") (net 1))
 (segment (start 185.93 76.708) (end 185.93 76.72857) (width 0.25) (layer "F.Cu") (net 1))
 (segment (start 184.05452 77.40252) (end 183.36 76.708) (width 0.25) (layer "F.Cu") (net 1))
 (segment (start 178.38548 77.39252) (end 176.931511 78.846489) (width 0.25) (layer "F.Cu") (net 2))
 (segment (start 182.4 76.708) (end 181.71548 77.39252) (width 0.25) (layer "F.Cu") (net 2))
 (segment (start 181.71548 77.39252) (end 178.38548 77.39252) (width 0.25) (layer "F.Cu") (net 2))
 (segment (start 182.4 76.708) (end 182.4 74.958) (width 0.25) (layer "F.Cu") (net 2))
 (segment (start 182.372 76.708) (end 182.4 76.708) (width 0.25) (layer "F.Cu") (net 2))
 (segment (start 173.312 80.18) (end 172.974 80.18) (width 0.25) (layer "F.Cu") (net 2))
 (segment (start 182.4 74.958) (end 182.372 74.93) (width 0.25) (layer "F.Cu") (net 2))
 (segment (start 174.645511 78.846489) (end 173.312 80.18) (width 0.25) (layer "F.Cu") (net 2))
 (segment (start 176.931511 78.846489) (end 174.645511 78.846489) (width 0.25) (layer "F.Cu") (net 2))
 (segment (start 179.86 75.09) (end 180.02 74.93) (width 0.25) (layer "F.Cu") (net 6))
 (segment (start 179.86 76.708) (end 179.86 75.09) (width 0.25) (layer "F.Cu") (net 6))
 (segment (start 189.926 71.5783) (end 189.23 70.8823) (width 0.5) (layer "F.Cu") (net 5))
 (segment (start 182.246 69.62) (end 182.778 69.088) (width 0.5) (layer "F.Cu") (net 7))
 (segment (start 181.966 69.34) (end 180.086 69.34) (width 0.5) (layer "F.Cu") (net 7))
 (segment (start 182.246 69.62) (end 181.966 69.34) (width 0.5) (layer "F.Cu") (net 7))
 (segment (start 182.778 69.088) (end 187.734 69.088) (width 0.5) (layer "F.Cu") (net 7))
 (segment (start 189.23 80.8823) (end 190.3563 80.8823) (width 0.25) (layer "F.Cu") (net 4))
 (segment (start 190.3563 80.8823) (end 190.754 81.28) (width 0.25) (layer "F.Cu") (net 4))
 (segment (start 189.23 80.8823) (end 176.8727 80.8823) (width 0.5) (layer "B.Cu") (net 4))
 (segment (start 176.8727 80.8823) (end 176.784 80.971) (width 0.5) (layer "B.Cu") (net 4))
 (segment (start 169.41 72.64) (end 169.414 72.644) (width 0.25) (layer "F.Cu") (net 8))
 (segment (start 169.41 70.282) (end 169.41 72.64) (width 0.25) (layer "F.Cu") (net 8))
 (segment (start 173.01 75.382) (end 175.321489 73.070511) (width 0.25) (layer "F.Cu") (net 9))
 (segment (start 179.128919 73.070511) (end 180.06543 72.134) (width 0.25) (layer "F.Cu") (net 9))
 (segment (start 175.321489 73.070511) (end 179.128919 73.070511) (width 0.25) (layer "F.Cu") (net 9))
 (segment (start 180.06543 72.134) (end 180.086 72.134) (width 0.25) (layer "F.Cu") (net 9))
 (segment (start 180.086 72.134) (end 180.086 70.36) (width 0.25) (layer "F.Cu") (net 9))
 (segment (start 169.926 77.724) (end 169.926 78.4075) (width 0.5) (layer "F.Cu") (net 13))
 (segment (start 169.926 78.4075) (end 166.7995 81.534) (width 0.5) (layer "F.Cu") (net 13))
 (via (at 166.7995 81.534) (size 0.8) (drill 0.4) (layers "F.Cu" "B.Cu") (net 13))
 (via (at 169.926 77.724) (size 0.8) (drill 0.4) (layers "F.Cu" "B.Cu") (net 13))
 (segment (start 176.8727 75.8823) (end 176.784 75.971) (width 0.5) (layer "B.Cu") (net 13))
 (segment (start 175.034001 77.720999) (end 169.929001 77.720999) (width 0.5) (layer "B.Cu") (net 13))
 (segment (start 176.784 75.971) (end 175.034001 77.720999) (width 0.5) (layer "B.Cu") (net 13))
 (segment (start 169.929001 77.720999) (end 169.926 77.724) (width 0.5) (layer "B.Cu") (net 13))
 (segment (start 189.23 75.8823) (end 176.8727 75.8823) (width 0.5) (layer "B.Cu") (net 13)))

